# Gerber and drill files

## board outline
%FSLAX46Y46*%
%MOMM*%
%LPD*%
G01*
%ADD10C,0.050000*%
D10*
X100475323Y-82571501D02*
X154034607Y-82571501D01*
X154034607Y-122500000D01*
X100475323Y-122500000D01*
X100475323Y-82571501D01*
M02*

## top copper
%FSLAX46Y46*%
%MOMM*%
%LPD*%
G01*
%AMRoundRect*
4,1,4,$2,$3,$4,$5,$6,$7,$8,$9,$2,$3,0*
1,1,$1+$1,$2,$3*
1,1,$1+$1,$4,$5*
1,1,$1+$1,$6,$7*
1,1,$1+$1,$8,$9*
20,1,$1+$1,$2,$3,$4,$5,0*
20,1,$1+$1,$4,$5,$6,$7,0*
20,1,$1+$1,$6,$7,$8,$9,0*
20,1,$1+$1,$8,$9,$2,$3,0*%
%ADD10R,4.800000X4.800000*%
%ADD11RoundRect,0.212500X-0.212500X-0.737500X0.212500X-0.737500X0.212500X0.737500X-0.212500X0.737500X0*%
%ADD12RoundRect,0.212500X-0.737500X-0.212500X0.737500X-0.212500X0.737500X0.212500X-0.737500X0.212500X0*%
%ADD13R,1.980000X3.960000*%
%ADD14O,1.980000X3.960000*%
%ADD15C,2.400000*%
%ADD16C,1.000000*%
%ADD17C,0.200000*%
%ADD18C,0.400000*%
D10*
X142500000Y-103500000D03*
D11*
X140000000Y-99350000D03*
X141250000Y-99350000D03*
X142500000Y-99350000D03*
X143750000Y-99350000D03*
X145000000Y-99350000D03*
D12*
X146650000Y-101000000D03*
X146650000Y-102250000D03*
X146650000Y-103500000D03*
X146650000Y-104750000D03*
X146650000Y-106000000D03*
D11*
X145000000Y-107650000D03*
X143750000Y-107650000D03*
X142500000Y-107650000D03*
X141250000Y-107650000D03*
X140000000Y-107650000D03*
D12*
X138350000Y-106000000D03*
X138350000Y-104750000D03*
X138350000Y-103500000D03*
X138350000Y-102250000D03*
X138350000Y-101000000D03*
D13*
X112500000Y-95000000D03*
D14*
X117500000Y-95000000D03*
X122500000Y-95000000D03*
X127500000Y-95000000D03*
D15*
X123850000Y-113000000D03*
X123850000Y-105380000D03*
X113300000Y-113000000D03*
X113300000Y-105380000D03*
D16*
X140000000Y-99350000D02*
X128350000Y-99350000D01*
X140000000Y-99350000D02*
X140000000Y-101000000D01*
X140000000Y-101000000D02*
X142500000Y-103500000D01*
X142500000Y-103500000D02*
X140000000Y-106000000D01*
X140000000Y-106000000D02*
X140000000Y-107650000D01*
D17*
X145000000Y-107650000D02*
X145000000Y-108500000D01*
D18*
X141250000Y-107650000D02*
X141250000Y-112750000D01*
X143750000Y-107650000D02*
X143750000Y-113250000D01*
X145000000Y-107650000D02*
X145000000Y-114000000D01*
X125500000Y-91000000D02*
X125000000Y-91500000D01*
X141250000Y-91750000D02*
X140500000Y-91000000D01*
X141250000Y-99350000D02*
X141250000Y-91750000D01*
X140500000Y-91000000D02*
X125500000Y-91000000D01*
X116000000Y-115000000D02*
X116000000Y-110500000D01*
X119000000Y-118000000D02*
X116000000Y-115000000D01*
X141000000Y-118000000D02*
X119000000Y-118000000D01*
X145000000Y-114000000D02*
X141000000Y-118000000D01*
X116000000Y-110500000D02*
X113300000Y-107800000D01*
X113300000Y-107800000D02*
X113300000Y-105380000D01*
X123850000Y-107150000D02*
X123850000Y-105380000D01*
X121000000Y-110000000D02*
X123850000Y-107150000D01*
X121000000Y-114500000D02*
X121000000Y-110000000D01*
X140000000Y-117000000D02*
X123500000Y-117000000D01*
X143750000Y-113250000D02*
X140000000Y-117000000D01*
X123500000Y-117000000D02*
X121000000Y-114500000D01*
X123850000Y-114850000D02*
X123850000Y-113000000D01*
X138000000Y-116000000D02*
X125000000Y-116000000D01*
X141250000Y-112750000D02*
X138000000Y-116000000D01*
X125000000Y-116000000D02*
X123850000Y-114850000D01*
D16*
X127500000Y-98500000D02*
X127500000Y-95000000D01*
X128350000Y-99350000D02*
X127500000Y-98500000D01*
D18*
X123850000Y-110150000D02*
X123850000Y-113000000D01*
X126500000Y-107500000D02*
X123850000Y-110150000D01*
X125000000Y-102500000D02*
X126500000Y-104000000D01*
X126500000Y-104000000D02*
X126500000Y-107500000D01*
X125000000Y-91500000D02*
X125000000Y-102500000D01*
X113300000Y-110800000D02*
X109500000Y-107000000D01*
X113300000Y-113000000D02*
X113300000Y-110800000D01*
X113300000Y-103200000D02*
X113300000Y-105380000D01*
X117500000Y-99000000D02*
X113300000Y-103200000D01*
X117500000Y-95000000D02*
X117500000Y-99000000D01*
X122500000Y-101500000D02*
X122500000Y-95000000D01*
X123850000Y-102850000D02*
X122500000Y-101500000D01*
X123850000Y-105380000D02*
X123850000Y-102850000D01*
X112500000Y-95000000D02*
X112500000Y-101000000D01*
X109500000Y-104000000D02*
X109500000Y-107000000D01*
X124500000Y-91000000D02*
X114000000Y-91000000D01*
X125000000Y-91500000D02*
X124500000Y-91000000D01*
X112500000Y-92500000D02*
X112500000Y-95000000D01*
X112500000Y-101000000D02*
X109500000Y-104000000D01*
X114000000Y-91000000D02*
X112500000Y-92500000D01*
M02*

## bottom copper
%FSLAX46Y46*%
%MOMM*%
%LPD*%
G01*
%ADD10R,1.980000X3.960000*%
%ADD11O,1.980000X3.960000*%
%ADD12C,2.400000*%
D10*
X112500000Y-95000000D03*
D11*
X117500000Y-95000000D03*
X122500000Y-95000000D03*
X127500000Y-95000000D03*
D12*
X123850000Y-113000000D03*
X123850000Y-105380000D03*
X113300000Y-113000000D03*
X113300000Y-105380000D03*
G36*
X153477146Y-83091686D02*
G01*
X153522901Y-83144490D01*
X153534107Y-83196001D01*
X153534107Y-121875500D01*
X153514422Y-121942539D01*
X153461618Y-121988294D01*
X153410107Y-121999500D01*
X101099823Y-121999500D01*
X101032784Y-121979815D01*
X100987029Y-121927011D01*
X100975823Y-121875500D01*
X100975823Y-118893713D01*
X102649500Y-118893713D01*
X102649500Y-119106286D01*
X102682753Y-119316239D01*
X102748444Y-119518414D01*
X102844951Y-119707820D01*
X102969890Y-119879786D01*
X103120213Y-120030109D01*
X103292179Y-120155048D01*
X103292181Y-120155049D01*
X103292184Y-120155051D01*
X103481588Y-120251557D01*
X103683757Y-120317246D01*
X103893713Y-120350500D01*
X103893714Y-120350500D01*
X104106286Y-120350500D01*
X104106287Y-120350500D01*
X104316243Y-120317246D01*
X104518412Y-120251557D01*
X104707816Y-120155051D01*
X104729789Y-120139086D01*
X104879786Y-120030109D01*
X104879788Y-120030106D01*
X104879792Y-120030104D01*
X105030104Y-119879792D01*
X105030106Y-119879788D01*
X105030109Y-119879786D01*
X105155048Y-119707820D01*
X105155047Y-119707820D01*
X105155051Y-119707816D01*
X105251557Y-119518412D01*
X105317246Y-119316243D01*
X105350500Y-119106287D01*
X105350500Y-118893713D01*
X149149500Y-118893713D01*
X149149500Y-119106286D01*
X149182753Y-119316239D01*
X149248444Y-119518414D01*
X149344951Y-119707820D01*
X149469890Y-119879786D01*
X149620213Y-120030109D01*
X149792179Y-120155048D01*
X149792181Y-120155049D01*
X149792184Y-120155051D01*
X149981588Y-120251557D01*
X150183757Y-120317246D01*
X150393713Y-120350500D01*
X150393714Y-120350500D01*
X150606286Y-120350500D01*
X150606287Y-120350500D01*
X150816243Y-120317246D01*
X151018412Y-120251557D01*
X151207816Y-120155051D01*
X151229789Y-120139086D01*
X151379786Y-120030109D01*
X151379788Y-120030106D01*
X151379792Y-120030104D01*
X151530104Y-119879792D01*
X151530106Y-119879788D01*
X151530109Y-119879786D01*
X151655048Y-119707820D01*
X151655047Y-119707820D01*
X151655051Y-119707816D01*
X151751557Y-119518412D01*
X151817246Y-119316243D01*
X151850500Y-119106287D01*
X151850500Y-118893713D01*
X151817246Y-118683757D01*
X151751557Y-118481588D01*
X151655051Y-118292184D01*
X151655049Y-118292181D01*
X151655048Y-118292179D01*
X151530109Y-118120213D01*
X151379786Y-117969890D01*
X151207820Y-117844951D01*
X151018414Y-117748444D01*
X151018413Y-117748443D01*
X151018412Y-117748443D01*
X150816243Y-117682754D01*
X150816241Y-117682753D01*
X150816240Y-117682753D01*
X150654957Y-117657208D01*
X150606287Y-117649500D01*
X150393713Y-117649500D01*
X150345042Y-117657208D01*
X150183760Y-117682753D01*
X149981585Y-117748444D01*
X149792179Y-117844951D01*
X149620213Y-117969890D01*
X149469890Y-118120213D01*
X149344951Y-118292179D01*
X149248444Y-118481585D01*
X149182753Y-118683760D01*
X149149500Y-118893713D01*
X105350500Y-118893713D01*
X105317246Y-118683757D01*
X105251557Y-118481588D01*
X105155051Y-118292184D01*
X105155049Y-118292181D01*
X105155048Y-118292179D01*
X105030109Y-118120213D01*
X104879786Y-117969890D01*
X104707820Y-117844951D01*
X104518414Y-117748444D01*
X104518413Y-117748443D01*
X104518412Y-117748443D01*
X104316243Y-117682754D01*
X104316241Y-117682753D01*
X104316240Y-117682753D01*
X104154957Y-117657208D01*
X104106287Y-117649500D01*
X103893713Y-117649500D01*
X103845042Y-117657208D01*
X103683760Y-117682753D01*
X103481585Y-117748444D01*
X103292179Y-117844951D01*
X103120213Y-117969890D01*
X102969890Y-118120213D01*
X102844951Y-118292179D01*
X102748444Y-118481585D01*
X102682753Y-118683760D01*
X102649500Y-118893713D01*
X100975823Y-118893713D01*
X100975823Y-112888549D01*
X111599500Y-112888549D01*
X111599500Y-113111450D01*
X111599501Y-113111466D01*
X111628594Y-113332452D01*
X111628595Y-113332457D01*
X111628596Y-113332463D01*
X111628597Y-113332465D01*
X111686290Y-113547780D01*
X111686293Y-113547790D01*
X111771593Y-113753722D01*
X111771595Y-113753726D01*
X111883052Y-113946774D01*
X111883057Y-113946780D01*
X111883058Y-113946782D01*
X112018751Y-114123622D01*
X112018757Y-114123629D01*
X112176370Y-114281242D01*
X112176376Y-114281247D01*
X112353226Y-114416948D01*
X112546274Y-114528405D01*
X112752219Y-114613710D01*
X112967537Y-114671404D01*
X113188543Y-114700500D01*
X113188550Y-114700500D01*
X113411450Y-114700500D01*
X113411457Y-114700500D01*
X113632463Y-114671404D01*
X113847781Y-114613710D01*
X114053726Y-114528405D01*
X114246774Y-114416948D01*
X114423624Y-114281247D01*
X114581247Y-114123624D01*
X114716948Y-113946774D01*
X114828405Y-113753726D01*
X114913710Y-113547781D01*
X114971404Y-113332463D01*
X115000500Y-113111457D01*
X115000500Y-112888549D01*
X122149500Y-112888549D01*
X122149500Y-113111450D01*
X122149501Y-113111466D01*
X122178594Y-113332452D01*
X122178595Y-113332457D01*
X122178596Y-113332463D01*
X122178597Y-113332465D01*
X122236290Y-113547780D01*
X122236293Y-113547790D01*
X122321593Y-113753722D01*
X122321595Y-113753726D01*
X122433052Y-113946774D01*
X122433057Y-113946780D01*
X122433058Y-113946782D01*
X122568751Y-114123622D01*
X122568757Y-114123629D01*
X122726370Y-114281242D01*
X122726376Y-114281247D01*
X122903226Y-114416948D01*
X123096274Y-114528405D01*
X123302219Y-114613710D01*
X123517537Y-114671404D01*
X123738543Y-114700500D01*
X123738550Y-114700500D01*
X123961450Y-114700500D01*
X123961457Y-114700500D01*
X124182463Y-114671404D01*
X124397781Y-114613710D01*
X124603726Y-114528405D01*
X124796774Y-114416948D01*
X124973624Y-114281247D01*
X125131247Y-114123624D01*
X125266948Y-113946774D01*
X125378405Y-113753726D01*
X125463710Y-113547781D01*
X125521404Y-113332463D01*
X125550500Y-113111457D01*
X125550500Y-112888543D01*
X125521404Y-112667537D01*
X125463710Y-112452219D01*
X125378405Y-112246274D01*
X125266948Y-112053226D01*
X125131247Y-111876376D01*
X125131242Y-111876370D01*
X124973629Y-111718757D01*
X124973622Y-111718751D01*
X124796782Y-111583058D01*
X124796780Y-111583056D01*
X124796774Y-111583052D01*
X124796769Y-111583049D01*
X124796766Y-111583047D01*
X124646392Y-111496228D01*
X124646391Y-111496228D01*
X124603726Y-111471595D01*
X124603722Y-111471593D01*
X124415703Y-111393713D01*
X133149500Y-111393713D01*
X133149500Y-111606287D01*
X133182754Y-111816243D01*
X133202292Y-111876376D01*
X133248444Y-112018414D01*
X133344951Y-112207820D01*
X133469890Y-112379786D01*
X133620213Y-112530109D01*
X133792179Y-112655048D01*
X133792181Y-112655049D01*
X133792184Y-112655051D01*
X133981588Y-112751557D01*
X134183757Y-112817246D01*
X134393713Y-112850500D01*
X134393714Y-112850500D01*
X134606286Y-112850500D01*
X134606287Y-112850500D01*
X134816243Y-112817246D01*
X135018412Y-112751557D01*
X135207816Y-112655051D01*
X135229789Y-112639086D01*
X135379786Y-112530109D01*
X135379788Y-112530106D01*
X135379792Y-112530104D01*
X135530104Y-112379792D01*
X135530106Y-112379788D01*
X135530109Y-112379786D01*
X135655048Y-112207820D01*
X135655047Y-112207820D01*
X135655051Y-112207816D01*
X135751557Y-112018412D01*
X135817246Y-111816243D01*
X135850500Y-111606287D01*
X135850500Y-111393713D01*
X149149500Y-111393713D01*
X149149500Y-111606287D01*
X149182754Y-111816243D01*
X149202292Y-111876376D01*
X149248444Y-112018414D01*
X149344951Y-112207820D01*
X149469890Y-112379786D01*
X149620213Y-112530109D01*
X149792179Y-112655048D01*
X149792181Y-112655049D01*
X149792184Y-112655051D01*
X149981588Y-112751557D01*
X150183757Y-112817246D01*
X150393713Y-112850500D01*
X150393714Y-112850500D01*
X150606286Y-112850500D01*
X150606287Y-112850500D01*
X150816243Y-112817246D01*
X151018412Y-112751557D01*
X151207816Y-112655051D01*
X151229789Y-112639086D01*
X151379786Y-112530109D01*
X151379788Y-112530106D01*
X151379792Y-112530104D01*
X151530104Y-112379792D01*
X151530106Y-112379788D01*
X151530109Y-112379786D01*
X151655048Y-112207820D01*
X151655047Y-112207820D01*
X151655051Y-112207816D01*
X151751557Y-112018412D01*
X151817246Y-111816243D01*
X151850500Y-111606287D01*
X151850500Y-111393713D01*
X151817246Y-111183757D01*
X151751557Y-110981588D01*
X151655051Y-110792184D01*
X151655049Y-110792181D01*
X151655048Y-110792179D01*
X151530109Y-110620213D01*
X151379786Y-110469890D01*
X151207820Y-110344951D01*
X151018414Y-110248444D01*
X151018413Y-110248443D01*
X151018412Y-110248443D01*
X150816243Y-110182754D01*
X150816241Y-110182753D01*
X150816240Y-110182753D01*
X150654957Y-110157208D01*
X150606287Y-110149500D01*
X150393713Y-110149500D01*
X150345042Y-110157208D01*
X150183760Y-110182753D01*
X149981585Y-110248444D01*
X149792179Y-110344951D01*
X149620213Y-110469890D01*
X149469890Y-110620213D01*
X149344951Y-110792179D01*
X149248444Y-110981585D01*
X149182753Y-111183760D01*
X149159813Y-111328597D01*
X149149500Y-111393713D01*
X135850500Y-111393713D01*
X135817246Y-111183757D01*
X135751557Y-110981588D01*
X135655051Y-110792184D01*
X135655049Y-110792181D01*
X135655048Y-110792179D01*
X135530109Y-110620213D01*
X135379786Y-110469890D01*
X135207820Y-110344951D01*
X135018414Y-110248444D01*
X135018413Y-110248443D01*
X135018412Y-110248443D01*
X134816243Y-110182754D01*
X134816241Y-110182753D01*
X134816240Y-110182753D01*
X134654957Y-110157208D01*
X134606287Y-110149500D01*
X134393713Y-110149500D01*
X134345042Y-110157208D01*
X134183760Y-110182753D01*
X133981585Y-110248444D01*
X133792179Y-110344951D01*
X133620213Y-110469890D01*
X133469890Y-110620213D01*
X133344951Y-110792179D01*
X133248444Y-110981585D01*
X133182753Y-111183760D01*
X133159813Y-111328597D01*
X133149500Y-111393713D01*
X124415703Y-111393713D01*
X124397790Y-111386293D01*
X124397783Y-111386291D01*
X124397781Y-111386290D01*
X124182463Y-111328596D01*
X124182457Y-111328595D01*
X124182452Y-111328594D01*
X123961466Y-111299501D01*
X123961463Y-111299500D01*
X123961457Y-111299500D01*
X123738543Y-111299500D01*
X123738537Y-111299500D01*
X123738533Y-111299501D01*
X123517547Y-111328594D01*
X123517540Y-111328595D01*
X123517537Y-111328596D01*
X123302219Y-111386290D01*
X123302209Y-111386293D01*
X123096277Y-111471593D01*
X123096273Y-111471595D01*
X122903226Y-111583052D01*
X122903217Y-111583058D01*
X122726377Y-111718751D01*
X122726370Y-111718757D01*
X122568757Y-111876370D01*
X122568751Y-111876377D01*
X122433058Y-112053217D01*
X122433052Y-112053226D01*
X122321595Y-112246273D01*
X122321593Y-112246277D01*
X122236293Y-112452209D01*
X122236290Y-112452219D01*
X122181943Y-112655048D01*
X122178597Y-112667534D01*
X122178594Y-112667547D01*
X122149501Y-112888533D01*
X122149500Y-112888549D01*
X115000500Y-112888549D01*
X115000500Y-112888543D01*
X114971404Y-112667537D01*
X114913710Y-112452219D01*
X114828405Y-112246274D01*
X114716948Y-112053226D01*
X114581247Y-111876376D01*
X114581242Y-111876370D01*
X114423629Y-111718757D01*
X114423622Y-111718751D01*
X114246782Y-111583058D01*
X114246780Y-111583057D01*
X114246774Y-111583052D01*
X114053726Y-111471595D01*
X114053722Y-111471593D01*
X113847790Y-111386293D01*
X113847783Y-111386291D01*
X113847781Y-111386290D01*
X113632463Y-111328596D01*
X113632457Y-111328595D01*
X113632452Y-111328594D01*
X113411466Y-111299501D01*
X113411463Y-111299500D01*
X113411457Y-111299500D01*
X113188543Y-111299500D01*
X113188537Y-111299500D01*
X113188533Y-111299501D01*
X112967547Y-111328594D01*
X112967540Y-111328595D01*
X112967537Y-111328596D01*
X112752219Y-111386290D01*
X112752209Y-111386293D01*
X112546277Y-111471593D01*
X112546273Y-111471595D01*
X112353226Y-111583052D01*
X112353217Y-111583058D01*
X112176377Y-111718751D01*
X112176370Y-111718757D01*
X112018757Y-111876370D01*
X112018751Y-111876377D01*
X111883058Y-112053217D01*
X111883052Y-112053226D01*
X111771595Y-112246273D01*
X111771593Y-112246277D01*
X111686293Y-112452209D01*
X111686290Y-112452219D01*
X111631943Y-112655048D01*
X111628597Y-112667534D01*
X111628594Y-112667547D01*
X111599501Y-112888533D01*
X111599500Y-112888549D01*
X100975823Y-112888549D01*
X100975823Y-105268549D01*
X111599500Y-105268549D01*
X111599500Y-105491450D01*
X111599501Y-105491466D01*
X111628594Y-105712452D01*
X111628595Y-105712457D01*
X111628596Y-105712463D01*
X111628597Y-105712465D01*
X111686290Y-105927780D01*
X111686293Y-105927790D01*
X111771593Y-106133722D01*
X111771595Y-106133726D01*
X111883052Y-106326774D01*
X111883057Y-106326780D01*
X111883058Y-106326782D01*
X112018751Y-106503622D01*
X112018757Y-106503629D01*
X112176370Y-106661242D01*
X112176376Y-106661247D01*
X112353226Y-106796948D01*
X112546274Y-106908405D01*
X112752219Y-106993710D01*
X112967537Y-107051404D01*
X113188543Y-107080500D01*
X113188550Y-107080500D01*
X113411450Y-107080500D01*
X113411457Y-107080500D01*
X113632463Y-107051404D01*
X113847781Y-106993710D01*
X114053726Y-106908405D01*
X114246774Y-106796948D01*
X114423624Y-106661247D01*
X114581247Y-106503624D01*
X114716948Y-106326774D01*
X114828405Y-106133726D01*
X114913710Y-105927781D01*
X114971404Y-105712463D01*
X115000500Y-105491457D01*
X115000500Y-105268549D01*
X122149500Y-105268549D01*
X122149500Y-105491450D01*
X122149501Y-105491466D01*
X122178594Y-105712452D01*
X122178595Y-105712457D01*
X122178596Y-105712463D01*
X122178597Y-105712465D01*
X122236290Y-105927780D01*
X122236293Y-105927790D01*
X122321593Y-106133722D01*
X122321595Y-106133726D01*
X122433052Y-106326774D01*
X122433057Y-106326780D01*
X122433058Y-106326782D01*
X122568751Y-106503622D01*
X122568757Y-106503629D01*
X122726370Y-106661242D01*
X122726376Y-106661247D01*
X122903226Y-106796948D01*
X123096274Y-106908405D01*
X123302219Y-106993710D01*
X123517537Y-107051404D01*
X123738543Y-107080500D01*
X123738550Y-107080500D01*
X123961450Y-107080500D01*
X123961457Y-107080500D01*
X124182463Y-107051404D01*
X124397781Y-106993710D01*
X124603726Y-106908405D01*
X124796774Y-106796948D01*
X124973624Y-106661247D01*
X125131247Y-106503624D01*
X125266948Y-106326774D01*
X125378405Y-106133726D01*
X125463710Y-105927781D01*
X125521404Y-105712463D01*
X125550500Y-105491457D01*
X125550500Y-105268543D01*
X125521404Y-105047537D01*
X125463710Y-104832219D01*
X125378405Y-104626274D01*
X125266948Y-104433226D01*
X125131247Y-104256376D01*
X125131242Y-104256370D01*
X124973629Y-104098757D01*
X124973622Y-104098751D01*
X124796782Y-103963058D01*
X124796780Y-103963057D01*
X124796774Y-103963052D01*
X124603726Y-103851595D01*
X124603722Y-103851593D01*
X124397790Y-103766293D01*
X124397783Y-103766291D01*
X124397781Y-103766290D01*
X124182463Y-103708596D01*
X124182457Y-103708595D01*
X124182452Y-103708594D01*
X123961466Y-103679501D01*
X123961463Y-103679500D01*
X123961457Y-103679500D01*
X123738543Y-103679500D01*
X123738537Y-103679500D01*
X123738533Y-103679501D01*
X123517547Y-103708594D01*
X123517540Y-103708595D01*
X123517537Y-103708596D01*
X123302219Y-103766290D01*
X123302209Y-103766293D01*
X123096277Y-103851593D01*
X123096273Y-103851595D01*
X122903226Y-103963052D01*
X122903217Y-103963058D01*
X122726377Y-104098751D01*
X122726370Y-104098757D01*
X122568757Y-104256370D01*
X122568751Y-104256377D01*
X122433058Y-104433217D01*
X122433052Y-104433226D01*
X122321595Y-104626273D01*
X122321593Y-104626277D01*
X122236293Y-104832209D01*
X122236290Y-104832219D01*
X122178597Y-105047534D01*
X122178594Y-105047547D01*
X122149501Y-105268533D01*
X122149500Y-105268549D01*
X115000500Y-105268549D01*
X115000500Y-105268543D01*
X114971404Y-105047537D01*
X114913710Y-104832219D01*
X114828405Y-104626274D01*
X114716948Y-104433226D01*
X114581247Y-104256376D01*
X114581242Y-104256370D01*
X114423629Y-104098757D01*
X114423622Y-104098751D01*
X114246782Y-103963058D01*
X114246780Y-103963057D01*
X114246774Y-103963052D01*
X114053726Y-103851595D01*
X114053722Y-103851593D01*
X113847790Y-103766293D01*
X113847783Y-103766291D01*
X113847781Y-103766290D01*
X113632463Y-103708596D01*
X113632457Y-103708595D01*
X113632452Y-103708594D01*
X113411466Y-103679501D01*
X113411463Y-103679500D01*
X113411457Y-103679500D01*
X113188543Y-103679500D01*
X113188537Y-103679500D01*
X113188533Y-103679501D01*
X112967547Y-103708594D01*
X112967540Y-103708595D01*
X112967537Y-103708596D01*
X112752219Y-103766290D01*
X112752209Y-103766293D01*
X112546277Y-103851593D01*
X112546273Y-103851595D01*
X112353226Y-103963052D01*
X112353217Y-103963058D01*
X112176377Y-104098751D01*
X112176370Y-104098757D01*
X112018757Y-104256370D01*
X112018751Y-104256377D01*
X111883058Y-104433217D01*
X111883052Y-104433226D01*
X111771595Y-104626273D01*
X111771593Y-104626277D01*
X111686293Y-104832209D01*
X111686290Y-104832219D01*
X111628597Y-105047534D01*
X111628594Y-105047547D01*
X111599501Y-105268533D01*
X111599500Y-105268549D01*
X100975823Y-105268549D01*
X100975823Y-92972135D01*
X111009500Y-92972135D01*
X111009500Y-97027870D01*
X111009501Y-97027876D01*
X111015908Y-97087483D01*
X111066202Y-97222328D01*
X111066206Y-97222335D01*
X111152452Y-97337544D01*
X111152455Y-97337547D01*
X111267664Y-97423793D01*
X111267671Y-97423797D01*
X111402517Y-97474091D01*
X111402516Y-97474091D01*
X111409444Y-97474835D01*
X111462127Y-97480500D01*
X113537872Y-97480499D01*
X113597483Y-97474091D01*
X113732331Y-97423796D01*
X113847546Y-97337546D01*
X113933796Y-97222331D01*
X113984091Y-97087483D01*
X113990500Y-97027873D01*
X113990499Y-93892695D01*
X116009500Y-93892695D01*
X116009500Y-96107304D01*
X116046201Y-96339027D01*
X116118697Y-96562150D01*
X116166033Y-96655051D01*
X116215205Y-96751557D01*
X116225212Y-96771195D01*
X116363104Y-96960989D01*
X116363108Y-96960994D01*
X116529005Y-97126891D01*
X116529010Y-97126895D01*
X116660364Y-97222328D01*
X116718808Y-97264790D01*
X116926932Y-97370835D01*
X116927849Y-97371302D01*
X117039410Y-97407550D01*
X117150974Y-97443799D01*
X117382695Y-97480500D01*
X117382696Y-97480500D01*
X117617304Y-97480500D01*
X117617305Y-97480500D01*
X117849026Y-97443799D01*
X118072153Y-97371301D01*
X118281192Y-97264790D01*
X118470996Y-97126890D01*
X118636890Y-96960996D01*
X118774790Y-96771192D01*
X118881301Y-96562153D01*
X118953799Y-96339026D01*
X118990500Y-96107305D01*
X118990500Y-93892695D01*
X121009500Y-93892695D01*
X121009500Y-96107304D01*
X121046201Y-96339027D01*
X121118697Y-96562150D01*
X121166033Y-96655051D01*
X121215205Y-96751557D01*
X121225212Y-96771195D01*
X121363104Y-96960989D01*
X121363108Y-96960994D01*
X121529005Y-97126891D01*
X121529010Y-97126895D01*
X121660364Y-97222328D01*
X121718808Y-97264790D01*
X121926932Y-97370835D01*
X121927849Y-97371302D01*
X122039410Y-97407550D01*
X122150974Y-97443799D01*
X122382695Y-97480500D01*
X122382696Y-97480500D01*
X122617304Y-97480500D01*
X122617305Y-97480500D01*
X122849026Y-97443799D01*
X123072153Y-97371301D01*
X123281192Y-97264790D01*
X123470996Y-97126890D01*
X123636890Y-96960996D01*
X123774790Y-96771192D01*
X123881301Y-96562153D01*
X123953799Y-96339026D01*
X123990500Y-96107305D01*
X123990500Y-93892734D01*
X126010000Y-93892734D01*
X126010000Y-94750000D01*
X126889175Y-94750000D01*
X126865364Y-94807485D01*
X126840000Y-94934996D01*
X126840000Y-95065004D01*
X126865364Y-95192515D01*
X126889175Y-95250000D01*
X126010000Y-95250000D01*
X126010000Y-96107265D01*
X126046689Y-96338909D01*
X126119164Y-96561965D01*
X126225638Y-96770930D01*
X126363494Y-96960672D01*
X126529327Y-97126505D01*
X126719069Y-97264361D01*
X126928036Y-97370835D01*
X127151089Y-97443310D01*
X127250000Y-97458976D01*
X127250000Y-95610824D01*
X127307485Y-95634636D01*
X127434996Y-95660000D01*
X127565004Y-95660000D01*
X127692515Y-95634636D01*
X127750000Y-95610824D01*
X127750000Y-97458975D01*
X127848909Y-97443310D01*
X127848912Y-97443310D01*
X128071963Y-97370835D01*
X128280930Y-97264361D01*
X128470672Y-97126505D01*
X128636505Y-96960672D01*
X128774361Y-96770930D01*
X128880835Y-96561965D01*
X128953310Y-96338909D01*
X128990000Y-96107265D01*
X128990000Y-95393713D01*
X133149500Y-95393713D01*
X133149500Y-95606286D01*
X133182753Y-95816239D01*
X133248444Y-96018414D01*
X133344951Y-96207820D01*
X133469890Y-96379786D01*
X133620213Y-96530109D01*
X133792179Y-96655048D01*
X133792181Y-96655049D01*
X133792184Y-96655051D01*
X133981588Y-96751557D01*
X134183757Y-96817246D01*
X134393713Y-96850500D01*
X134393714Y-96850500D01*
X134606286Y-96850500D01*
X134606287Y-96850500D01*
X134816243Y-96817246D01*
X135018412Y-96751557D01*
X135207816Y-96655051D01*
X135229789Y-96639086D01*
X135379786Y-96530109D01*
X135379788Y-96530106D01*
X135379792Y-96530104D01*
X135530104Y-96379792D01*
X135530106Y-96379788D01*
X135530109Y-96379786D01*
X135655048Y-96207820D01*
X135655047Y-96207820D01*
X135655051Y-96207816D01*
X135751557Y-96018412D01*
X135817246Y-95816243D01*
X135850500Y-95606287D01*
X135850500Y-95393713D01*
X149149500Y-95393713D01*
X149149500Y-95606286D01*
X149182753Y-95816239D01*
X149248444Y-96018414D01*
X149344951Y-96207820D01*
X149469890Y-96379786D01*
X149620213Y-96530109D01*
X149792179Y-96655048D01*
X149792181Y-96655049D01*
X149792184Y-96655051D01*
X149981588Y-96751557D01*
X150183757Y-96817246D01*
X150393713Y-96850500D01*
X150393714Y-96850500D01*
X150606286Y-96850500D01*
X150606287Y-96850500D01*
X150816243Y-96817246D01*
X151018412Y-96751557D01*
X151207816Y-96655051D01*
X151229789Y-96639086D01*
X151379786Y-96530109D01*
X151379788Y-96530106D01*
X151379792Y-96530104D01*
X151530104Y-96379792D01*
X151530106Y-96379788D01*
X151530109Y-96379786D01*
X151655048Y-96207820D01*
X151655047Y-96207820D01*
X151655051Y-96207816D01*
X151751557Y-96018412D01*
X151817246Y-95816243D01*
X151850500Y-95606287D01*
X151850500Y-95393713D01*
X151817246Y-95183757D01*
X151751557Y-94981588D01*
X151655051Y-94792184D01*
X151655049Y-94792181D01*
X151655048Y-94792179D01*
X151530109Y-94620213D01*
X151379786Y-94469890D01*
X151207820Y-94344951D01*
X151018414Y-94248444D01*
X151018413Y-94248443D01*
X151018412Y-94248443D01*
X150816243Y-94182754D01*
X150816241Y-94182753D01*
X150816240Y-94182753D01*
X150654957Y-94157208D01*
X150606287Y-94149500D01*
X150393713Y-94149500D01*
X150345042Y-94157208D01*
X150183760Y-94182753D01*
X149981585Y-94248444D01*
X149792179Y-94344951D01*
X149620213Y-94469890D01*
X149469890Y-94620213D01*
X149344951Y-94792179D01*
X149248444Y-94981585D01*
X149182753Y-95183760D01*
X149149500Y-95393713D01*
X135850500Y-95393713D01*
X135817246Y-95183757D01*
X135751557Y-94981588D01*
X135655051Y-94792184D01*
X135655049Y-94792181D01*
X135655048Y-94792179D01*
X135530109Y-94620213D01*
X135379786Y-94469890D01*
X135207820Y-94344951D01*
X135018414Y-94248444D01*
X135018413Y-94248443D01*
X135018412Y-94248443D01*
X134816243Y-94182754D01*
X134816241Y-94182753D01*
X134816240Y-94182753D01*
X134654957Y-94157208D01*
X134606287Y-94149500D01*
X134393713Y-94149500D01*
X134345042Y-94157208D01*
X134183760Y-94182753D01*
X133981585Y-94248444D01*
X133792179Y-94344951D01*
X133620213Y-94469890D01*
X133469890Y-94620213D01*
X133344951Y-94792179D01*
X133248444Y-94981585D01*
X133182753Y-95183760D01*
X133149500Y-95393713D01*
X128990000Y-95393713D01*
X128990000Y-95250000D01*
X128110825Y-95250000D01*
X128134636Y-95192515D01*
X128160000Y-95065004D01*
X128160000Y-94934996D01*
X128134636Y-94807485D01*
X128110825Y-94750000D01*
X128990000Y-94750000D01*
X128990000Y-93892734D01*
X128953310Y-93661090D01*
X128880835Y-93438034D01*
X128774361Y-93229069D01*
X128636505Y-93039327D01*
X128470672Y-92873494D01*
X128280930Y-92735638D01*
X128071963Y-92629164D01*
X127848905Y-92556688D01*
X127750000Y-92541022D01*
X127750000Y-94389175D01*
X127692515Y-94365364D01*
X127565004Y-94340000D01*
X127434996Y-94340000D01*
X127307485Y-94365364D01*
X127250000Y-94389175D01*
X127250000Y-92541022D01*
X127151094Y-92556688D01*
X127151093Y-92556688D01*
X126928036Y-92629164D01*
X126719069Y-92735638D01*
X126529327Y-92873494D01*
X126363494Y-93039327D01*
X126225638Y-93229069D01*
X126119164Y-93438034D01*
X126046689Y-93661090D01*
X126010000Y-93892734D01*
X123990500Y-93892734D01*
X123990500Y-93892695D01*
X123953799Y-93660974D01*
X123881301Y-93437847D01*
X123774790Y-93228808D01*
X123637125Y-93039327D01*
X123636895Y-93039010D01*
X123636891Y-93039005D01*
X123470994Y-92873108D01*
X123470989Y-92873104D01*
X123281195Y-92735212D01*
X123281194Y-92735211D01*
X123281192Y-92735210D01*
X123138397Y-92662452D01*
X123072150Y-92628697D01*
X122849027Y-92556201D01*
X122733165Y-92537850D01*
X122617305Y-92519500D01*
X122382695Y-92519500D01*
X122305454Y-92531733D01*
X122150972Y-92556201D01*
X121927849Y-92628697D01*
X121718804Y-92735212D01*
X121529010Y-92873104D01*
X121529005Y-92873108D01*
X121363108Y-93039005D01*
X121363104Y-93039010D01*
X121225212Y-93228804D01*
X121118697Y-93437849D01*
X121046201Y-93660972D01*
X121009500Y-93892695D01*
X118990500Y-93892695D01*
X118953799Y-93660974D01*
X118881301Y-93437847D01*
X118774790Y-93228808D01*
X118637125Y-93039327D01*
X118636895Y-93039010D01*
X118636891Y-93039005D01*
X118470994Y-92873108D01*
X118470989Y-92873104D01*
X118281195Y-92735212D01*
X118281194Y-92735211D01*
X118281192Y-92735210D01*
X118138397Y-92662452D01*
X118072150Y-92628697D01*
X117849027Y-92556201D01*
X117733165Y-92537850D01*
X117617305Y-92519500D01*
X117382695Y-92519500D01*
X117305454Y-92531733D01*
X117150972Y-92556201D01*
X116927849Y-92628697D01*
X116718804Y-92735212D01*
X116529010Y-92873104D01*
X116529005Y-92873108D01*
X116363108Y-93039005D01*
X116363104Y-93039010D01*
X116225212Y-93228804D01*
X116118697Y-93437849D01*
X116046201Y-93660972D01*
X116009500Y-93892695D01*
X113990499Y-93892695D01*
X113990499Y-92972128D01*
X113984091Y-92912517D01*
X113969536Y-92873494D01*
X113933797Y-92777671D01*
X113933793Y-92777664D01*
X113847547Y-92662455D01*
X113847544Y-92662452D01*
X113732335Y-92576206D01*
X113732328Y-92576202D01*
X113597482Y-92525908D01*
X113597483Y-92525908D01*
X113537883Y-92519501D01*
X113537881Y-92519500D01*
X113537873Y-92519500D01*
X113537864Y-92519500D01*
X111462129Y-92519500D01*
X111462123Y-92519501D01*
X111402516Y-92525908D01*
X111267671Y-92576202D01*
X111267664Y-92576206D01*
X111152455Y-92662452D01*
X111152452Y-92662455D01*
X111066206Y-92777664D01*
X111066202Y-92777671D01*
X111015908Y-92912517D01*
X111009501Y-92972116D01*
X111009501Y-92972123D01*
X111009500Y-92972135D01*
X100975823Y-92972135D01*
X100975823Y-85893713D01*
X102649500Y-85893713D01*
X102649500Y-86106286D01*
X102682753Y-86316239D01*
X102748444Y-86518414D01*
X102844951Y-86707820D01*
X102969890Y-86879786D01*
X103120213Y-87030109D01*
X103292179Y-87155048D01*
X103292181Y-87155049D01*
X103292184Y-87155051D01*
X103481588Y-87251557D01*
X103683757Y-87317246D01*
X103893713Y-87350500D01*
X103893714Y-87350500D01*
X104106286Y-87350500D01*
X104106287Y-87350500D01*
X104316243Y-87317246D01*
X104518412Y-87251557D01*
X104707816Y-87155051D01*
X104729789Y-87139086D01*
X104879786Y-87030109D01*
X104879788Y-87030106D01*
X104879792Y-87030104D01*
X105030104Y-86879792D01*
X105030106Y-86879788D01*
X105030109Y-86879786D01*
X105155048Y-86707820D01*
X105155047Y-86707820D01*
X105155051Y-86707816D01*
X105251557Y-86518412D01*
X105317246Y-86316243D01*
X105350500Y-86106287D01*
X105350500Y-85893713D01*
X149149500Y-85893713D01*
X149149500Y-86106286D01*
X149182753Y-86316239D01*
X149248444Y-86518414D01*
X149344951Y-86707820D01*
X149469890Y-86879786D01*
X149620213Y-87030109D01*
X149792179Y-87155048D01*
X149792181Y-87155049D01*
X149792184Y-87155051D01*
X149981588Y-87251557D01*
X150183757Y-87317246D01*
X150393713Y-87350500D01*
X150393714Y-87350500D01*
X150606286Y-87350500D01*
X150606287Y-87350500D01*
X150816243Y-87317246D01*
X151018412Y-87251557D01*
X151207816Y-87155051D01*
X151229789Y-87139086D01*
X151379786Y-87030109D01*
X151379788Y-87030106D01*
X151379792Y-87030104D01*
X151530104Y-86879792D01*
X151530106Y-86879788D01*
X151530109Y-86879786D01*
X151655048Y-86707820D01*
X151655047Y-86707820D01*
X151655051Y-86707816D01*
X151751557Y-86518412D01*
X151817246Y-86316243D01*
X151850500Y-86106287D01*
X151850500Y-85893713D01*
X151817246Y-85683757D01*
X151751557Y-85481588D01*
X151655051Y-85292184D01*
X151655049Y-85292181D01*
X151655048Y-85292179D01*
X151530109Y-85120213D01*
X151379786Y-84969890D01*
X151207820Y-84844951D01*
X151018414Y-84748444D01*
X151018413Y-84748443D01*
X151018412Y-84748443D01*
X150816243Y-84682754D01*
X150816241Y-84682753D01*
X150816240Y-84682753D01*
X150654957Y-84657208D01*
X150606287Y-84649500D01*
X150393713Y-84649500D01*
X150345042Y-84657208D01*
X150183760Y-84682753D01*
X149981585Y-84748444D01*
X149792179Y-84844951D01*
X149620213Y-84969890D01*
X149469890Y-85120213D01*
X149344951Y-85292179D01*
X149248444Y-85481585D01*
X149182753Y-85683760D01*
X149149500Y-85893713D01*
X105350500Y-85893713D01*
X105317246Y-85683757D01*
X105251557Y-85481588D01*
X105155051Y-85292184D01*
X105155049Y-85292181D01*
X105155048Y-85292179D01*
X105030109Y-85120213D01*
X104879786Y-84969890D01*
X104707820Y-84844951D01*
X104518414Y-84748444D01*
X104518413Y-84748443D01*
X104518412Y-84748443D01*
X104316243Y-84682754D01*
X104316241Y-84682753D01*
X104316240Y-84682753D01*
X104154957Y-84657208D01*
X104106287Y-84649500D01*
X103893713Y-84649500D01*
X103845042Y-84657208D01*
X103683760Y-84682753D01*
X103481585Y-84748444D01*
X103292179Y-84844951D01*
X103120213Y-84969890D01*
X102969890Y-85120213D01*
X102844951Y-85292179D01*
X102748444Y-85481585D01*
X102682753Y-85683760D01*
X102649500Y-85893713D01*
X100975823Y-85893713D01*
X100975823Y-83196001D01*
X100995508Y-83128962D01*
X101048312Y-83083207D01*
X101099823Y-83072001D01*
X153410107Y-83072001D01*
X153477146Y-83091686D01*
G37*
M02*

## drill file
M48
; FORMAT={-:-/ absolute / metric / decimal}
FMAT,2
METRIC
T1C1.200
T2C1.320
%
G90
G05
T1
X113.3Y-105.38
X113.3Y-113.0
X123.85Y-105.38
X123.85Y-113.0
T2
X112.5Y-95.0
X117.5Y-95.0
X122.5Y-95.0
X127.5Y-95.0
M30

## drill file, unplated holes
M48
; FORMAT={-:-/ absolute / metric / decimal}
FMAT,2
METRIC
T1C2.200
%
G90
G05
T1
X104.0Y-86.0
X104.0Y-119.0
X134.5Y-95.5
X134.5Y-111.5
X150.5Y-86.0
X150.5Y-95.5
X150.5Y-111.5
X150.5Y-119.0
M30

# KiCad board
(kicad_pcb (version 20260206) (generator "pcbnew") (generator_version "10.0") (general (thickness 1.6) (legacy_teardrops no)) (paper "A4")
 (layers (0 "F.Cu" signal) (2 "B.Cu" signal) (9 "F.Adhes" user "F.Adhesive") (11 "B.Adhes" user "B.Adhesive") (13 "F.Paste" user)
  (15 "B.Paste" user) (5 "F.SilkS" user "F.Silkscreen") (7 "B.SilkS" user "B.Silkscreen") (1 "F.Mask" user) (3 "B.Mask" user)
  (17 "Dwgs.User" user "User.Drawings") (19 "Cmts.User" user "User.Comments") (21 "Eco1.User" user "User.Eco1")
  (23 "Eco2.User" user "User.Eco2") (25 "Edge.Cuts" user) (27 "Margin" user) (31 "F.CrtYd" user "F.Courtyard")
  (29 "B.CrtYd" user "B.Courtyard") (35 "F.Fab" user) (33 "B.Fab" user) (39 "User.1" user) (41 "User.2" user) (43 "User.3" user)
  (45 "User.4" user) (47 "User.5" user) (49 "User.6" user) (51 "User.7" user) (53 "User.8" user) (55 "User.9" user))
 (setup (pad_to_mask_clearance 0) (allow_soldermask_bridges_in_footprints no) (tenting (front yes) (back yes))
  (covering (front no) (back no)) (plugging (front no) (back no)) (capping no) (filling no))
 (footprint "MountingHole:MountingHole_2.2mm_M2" (layer "F.Cu") (at 104 119)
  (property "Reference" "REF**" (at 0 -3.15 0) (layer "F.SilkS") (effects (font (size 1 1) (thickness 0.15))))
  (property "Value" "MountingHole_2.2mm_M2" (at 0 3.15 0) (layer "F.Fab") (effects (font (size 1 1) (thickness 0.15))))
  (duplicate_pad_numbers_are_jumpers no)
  (pad "" np_thru_hole circle (at 0 0) (size 2.2 2.2) (drill 2.2) (layers "*.Cu" "*.Mask")))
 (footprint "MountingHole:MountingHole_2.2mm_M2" (layer "F.Cu") (at 150.5 111.5)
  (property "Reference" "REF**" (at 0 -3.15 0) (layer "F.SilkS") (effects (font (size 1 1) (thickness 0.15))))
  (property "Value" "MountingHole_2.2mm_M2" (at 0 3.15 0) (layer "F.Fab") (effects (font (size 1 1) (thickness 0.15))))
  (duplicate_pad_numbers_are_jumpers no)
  (pad "" np_thru_hole circle (at 0 0) (size 2.2 2.2) (drill 2.2) (layers "*.Cu" "*.Mask")))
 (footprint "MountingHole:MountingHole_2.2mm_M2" (layer "F.Cu") (at 150.5 86)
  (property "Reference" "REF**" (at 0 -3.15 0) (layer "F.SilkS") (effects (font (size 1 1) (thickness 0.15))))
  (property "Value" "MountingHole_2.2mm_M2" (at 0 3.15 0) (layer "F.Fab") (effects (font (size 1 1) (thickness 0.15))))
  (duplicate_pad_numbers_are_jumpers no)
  (pad "" np_thru_hole circle (at 0 0) (size 2.2 2.2) (drill 2.2) (layers "*.Cu" "*.Mask")))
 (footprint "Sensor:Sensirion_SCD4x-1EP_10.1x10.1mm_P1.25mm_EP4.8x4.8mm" (layer "F.Cu") (at 142.5 103.5)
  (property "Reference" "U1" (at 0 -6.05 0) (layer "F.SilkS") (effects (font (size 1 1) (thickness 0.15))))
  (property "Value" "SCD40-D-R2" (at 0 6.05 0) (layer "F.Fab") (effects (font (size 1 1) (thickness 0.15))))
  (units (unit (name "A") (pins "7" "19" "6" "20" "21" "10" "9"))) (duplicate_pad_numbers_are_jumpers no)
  (pad "" smd roundrect (at -1.2 -1.2) (size 1.93 1.93) (layers "F.Paste") (roundrect_rratio 0.129534))
  (pad "" smd roundrect (at -1.2 1.2) (size 1.93 1.93) (layers "F.Paste") (roundrect_rratio 0.129534))
  (pad "" smd roundrect (at 1.2 -1.2) (size 1.93 1.93) (layers "F.Paste") (roundrect_rratio 0.129534))
  (pad "" smd roundrect (at 1.2 1.2) (size 1.93 1.93) (layers "F.Paste") (roundrect_rratio 0.129534))
  (pad "1" smd roundrect (at -4.15 -2.5) (size 1.9 0.85) (layers "F.Cu" "F.Mask" "F.Paste") (roundrect_rratio 0.25))
  (pad "2" smd roundrect (at -4.15 -1.25) (size 1.9 0.85) (layers "F.Cu" "F.Mask" "F.Paste") (roundrect_rratio 0.25))
  (pad "3" smd roundrect (at -4.15 0) (size 1.9 0.85) (layers "F.Cu" "F.Mask" "F.Paste") (roundrect_rratio 0.25))
  (pad "4" smd roundrect (at -4.15 1.25) (size 1.9 0.85) (layers "F.Cu" "F.Mask" "F.Paste") (roundrect_rratio 0.25))
  (pad "5" smd roundrect (at -4.15 2.5) (size 1.9 0.85) (layers "F.Cu" "F.Mask" "F.Paste") (roundrect_rratio 0.25))
  (pad "6" smd roundrect (at -2.5 4.15) (size 0.85 1.9) (layers "F.Cu" "F.Mask" "F.Paste") (roundrect_rratio 0.25) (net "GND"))
  (pad "7" smd roundrect (at -1.25 4.15) (size 0.85 1.9) (layers "F.Cu" "F.Mask" "F.Paste") (roundrect_rratio 0.25) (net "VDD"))
  (pad "8" smd roundrect (at 0 4.15) (size 0.85 1.9) (layers "F.Cu" "F.Mask" "F.Paste") (roundrect_rratio 0.25))
  (pad "9" smd roundrect (at 1.25 4.15) (size 0.85 1.9) (layers "F.Cu" "F.Mask" "F.Paste") (roundrect_rratio 0.25) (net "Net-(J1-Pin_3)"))
  (pad "10" smd roundrect (at 2.5 4.15) (size 0.85 1.9) (layers "F.Cu" "F.Mask" "F.Paste") (roundrect_rratio 0.25) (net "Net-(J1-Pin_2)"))
  (pad "11" smd roundrect (at 4.15 2.5) (size 1.9 0.85) (layers "F.Cu" "F.Mask" "F.Paste") (roundrect_rratio 0.25))
  (pad "12" smd roundrect (at 4.15 1.25) (size 1.9 0.85) (layers "F.Cu" "F.Mask" "F.Paste") (roundrect_rratio 0.25))
  (pad "13" smd roundrect (at 4.15 0) (size 1.9 0.85) (layers "F.Cu" "F.Mask" "F.Paste") (roundrect_rratio 0.25))
  (pad "14" smd roundrect (at 4.15 -1.25) (size 1.9 0.85) (layers "F.Cu" "F.Mask" "F.Paste") (roundrect_rratio 0.25))
  (pad "15" smd roundrect (at 4.15 -2.5) (size 1.9 0.85) (layers "F.Cu" "F.Mask" "F.Paste") (roundrect_rratio 0.25))
  (pad "16" smd roundrect (at 2.5 -4.15) (size 0.85 1.9) (layers "F.Cu" "F.Mask" "F.Paste") (roundrect_rratio 0.25))
  (pad "17" smd roundrect (at 1.25 -4.15) (size 0.85 1.9) (layers "F.Cu" "F.Mask" "F.Paste") (roundrect_rratio 0.25))
  (pad "18" smd roundrect (at 0 -4.15) (size 0.85 1.9) (layers "F.Cu" "F.Mask" "F.Paste") (roundrect_rratio 0.25))
  (pad "19" smd roundrect (at -1.25 -4.15) (size 0.85 1.9) (layers "F.Cu" "F.Mask" "F.Paste") (roundrect_rratio 0.25) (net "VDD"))
  (pad "20" smd roundrect (at -2.5 -4.15) (size 0.85 1.9) (layers "F.Cu" "F.Mask" "F.Paste") (roundrect_rratio 0.25) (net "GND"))
  (pad "21" smd rect (at 0 0) (size 4.8 4.8) (layers "F.Cu" "F.Mask") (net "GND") (zone_connect 2)))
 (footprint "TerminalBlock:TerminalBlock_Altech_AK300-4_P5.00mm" (layer "F.Cu") (at 112.5 95)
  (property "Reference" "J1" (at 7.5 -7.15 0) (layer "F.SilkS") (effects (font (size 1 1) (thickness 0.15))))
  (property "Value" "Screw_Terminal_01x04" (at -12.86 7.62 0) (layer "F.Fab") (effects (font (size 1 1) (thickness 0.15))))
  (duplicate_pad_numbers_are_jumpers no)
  (pad "1" thru_hole rect (at 0 0) (size 1.98 3.96) (drill 1.32) (layers "*.Cu" "*.Mask") (remove_unused_layers no) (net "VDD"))
  (pad "2" thru_hole oval (at 5 0) (size 1.98 3.96) (drill 1.32) (layers "*.Cu" "*.Mask") (remove_unused_layers no) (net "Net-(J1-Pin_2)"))
  (pad "3" thru_hole oval (at 10 0) (size 1.98 3.96) (drill 1.32) (layers "*.Cu" "*.Mask") (remove_unused_layers no) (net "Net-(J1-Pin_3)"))
  (pad "4" thru_hole oval (at 15 0) (size 1.98 3.96) (drill 1.32) (layers "*.Cu" "*.Mask") (remove_unused_layers no) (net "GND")))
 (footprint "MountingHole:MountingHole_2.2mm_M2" (layer "F.Cu") (at 150.5 95.5)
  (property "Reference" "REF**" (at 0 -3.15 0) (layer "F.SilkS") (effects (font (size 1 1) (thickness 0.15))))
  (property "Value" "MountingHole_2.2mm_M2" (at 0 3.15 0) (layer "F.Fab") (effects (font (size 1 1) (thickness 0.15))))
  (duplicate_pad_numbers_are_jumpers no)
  (pad "" np_thru_hole circle (at 0 0) (size 2.2 2.2) (drill 2.2) (layers "*.Cu" "*.Mask")))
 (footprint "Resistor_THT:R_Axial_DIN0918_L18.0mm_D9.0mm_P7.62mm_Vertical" (layer "F.Cu") (at 123.85 113 90)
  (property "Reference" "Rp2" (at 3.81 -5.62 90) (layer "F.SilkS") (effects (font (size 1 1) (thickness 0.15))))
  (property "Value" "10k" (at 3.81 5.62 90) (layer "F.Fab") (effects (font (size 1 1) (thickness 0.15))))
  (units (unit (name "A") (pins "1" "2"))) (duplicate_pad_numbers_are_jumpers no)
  (pad "1" thru_hole circle (at 0 0 90) (size 2.4 2.4) (drill 1.2) (layers "*.Cu" "*.Mask") (remove_unused_layers no) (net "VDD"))
  (pad "2" thru_hole circle (at 7.62 0 90) (size 2.4 2.4) (drill 1.2) (layers "*.Cu" "*.Mask") (remove_unused_layers no)
   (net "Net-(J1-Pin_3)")))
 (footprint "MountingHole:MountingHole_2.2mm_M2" (layer "F.Cu") (at 150.5 119)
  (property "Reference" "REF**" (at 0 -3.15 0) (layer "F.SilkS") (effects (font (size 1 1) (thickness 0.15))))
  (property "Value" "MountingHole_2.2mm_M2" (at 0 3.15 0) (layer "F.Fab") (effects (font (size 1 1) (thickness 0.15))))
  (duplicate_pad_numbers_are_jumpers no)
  (pad "" np_thru_hole circle (at 0 0) (size 2.2 2.2) (drill 2.2) (layers "*.Cu" "*.Mask")))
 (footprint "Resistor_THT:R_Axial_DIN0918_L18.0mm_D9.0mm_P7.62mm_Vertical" (layer "F.Cu") (at 113.3 113 90)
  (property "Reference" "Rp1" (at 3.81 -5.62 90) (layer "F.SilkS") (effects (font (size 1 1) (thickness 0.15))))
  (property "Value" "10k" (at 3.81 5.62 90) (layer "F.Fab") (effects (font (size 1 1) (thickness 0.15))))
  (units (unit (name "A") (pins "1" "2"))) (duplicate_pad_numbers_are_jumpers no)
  (pad "1" thru_hole circle (at 0 0 90) (size 2.4 2.4) (drill 1.2) (layers "*.Cu" "*.Mask") (remove_unused_layers no) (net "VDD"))
  (pad "2" thru_hole circle (at 7.62 0 90) (size 2.4 2.4) (drill 1.2) (layers "*.Cu" "*.Mask") (remove_unused_layers no)
   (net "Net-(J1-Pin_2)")))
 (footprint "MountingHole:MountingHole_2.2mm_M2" (layer "F.Cu") (at 104 86)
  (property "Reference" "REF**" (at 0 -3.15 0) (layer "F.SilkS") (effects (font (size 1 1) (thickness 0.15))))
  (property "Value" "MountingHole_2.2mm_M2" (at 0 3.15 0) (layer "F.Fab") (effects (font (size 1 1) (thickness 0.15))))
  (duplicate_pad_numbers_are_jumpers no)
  (pad "" np_thru_hole circle (at 0 0) (size 2.2 2.2) (drill 2.2) (layers "*.Cu" "*.Mask")))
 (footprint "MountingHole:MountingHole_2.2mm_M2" (layer "F.Cu") (at 134.5 111.5)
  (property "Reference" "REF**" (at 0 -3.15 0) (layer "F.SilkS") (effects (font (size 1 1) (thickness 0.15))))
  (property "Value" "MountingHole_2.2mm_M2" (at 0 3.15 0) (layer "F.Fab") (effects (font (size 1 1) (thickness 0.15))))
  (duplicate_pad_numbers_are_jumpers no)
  (pad "" np_thru_hole circle (at 0 0) (size 2.2 2.2) (drill 2.2) (layers "*.Cu" "*.Mask")))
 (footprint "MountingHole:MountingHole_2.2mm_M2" (layer "F.Cu") (at 134.5 95.5)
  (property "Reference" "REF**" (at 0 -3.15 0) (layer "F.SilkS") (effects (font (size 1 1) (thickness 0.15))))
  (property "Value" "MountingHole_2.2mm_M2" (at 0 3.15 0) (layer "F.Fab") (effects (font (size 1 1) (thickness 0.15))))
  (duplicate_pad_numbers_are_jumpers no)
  (pad "" np_thru_hole circle (at 0 0) (size 2.2 2.2) (drill 2.2) (layers "*.Cu" "*.Mask")))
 (gr_rect (start 100.475323 82.571501) (end 154.034607 122.5) (stroke (width 0.05) (type default)) (fill no) (layer "Edge.Cuts"))
 (segment (start 140 101) (end 142.5 103.5) (width 1) (layer "F.Cu") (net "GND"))
 (segment (start 140 99.35) (end 140 101) (width 1) (layer "F.Cu") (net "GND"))
 (segment (start 140 99.35) (end 128.35 99.35) (width 1) (layer "F.Cu") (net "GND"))
 (segment (start 140 106) (end 140 107.65) (width 1) (layer "F.Cu") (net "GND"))
 (segment (start 142.5 103.5) (end 140 106) (width 1) (layer "F.Cu") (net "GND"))
 (segment (start 128.35 99.35) (end 127.5 98.5) (width 1) (layer "F.Cu") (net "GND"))
 (segment (start 127.5 98.5) (end 127.5 95) (width 1) (layer "F.Cu") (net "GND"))
 (segment (start 141.25 91.75) (end 140.5 91) (width 0.4) (layer "F.Cu") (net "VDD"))
 (segment (start 123.85 114.85) (end 123.85 113) (width 0.4) (layer "F.Cu") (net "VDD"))
 (segment (start 112.5 95) (end 112.5 101) (width 0.4) (layer "F.Cu") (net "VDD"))
 (segment (start 123.85 110.15) (end 123.85 113) (width 0.4) (layer "F.Cu") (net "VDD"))
 (segment (start 109.5 104) (end 109.5 107) (width 0.4) (layer "F.Cu") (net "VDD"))
 (segment (start 126.5 104) (end 126.5 107.5) (width 0.4) (layer "F.Cu") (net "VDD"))
 (segment (start 141.25 107.65) (end 141.25 112.75) (width 0.4) (layer "F.Cu") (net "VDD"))
 (segment (start 113.3 113) (end 113.3 110.8) (width 0.4) (layer "F.Cu") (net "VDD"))
 (segment (start 124.5 91) (end 114 91) (width 0.4) (layer "F.Cu") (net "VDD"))
 (segment (start 125 91.5) (end 124.5 91) (width 0.4) (layer "F.Cu") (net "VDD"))
 (segment (start 113.3 110.8) (end 109.5 107) (width 0.4) (layer "F.Cu") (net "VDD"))
 (segment (start 125 91.5) (end 125 102.5) (width 0.4) (layer "F.Cu") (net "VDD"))
 (segment (start 141.25 112.75) (end 138 116) (width 0.4) (layer "F.Cu") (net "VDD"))
 (segment (start 112.5 92.5) (end 112.5 95) (width 0.4) (layer "F.Cu") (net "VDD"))
 (segment (start 126.5 107.5) (end 123.85 110.15) (width 0.4) (layer "F.Cu") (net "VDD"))
 (segment (start 112.5 101) (end 109.5 104) (width 0.4) (layer "F.Cu") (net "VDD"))
 (segment (start 138 116) (end 125 116) (width 0.4) (layer "F.Cu") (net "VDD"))
 (segment (start 125.5 91) (end 125 91.5) (width 0.4) (layer "F.Cu") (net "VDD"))
 (segment (start 141.25 99.35) (end 141.25 91.75) (width 0.4) (layer "F.Cu") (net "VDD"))
 (segment (start 125 102.5) (end 126.5 104) (width 0.4) (layer "F.Cu") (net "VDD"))
 (segment (start 140.5 91) (end 125.5 91) (width 0.4) (layer "F.Cu") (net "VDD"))
 (segment (start 114 91) (end 112.5 92.5) (width 0.4) (layer "F.Cu") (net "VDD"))
 (segment (start 125 116) (end 123.85 114.85) (width 0.4) (layer "F.Cu") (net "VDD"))
 (segment (start 121 114.5) (end 121 110) (width 0.4) (layer "F.Cu") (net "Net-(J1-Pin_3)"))
 (segment (start 123.85 105.38) (end 123.85 102.85) (width 0.4) (layer "F.Cu") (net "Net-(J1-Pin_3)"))
 (segment (start 143.75 113.25) (end 140 117) (width 0.4) (layer "F.Cu") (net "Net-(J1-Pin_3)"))
 (segment (start 140 117) (end 123.5 117) (width 0.4) (layer "F.Cu") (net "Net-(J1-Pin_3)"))
 (segment (start 143.75 107.65) (end 143.75 113.25) (width 0.4) (layer "F.Cu") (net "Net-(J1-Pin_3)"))
 (segment (start 123.5 117) (end 121 114.5) (width 0.4) (layer "F.Cu") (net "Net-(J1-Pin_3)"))
 (segment (start 123.85 102.85) (end 122.5 101.5) (width 0.4) (layer "F.Cu") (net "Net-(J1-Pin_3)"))
 (segment (start 123.85 107.15) (end 123.85 105.38) (width 0.4) (layer "F.Cu") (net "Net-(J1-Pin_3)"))
 (segment (start 121 110) (end 123.85 107.15) (width 0.4) (layer "F.Cu") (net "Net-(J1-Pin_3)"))
 (segment (start 122.5 101.5) (end 122.5 95) (width 0.4) (layer "F.Cu") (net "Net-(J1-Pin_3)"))
 (segment (start 117.5 95) (end 117.5 99) (width 0.4) (layer "F.Cu") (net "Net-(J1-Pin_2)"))
 (segment (start 145 107.65) (end 145 114) (width 0.4) (layer "F.Cu") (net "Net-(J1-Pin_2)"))
 (segment (start 113.3 107.8) (end 113.3 105.38) (width 0.4) (layer "F.Cu") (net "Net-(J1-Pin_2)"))
 (segment (start 119 118) (end 116 115) (width 0.4) (layer "F.Cu") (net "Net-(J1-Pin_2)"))
 (segment (start 113.3 103.2) (end 113.3 105.38) (width 0.4) (layer "F.Cu") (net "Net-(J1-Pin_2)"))
 (segment (start 116 110.5) (end 113.3 107.8) (width 0.4) (layer "F.Cu") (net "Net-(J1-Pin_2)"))
 (segment (start 116 115) (end 116 110.5) (width 0.4) (layer "F.Cu") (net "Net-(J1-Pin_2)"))
 (segment (start 117.5 99) (end 113.3 103.2) (width 0.4) (layer "F.Cu") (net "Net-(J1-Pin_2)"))
 (segment (start 145 107.65) (end 145 108.5) (width 0.2) (layer "F.Cu") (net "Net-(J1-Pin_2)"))
 (segment (start 145 114) (end 141 118) (width 0.4) (layer "F.Cu") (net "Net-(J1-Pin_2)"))
 (segment (start 141 118) (end 119 118) (width 0.4) (layer "F.Cu") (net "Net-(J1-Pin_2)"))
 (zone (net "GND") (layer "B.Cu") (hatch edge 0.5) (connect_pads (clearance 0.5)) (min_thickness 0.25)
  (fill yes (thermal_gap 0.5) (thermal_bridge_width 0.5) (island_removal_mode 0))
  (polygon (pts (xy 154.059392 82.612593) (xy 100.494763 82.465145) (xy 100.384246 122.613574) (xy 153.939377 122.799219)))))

